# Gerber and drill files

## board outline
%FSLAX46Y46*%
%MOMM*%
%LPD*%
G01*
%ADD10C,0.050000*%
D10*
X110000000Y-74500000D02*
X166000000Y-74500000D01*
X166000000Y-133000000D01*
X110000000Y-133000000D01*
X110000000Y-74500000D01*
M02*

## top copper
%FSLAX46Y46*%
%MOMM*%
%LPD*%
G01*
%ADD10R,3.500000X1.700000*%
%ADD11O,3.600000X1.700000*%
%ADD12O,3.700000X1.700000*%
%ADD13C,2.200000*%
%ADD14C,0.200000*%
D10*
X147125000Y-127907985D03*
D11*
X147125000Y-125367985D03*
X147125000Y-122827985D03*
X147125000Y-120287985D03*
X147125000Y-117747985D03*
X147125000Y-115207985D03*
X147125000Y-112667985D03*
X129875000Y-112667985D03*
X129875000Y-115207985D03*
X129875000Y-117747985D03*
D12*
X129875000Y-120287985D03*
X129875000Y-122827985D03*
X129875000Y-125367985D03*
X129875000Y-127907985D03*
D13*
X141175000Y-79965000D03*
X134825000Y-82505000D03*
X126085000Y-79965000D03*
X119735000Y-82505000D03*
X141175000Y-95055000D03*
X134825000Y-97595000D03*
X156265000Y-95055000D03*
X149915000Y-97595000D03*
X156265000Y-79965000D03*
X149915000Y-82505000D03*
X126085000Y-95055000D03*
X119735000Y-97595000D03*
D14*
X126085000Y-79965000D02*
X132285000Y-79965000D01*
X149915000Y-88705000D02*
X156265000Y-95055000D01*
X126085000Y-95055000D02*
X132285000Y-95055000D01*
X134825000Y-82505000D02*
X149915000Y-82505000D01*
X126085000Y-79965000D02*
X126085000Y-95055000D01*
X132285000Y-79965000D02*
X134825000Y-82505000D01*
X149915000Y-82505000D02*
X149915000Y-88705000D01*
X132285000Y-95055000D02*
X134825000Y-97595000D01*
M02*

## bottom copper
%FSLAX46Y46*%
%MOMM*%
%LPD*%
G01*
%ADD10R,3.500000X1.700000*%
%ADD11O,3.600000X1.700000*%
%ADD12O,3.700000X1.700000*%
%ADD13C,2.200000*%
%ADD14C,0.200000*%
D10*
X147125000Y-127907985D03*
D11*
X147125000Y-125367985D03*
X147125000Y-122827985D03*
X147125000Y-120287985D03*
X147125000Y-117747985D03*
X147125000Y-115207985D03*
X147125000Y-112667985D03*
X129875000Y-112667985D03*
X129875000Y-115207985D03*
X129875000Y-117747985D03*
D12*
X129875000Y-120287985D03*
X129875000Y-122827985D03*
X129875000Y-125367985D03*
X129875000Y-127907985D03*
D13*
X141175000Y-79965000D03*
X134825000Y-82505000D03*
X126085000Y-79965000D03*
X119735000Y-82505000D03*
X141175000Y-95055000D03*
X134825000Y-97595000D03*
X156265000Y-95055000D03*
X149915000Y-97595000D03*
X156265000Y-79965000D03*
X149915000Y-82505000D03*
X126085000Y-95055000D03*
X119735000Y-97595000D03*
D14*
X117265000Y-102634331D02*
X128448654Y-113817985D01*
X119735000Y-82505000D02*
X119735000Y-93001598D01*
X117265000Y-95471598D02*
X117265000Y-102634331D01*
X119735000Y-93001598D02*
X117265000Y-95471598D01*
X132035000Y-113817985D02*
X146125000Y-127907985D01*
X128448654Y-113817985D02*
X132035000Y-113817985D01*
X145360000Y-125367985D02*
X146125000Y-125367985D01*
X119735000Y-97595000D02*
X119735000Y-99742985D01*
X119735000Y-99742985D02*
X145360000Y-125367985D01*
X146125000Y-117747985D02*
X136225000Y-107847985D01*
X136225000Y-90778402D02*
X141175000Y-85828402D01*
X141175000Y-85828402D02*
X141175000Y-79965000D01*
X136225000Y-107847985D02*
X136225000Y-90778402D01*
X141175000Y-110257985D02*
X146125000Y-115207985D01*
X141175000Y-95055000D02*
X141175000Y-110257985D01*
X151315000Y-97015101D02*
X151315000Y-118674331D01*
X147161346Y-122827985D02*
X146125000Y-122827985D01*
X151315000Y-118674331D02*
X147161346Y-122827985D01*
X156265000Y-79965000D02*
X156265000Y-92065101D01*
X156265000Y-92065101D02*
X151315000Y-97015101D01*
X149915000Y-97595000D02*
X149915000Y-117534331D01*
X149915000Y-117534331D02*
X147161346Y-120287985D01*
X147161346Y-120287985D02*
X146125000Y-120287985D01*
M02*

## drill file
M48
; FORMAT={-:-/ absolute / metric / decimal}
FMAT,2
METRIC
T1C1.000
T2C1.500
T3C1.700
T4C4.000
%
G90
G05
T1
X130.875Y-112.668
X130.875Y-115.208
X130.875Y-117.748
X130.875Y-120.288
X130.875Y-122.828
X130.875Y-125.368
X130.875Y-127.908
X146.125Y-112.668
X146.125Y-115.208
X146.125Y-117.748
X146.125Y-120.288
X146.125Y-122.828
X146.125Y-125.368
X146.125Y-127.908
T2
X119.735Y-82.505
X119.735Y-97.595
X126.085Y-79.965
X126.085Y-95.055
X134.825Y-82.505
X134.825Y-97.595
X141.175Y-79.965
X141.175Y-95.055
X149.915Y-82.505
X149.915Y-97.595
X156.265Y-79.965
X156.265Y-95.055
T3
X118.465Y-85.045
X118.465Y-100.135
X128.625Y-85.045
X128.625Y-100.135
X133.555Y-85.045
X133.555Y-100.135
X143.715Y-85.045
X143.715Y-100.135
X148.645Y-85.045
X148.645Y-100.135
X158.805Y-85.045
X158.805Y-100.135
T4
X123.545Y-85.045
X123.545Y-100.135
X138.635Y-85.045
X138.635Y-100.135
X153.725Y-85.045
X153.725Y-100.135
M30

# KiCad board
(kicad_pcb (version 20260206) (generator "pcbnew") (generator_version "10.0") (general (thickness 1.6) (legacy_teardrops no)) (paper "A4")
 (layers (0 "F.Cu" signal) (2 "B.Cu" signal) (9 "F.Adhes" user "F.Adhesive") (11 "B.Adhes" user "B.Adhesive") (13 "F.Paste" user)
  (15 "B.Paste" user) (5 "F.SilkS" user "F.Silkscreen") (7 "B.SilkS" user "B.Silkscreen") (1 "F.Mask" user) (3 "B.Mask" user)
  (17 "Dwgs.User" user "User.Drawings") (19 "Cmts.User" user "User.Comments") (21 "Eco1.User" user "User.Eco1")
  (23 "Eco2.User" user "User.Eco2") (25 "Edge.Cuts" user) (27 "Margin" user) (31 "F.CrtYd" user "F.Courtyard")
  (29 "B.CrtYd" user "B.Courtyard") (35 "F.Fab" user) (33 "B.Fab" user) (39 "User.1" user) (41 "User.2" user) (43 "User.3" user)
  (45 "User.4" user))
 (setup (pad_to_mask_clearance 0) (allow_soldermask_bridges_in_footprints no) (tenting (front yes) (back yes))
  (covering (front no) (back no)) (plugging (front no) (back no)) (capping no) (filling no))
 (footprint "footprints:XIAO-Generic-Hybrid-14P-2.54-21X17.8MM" (layer "F.Cu") (at 138.5 120.287985 180)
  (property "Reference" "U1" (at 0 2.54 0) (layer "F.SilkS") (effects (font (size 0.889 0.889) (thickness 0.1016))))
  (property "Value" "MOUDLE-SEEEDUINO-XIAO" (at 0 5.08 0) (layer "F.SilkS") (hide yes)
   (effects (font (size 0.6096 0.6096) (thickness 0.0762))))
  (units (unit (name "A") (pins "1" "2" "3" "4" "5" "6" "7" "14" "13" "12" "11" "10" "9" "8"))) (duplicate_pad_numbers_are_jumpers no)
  (pad "1" thru_hole rect (at -7.625 -7.62 180) (size 3.5 1.7) (drill 1 (offset -1 0)) (layers "*.Cu" "*.Mask") (remove_unused_layers no)
   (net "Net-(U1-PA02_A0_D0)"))
  (pad "2" thru_hole oval (at -7.625 -5.08 180) (size 3.6 1.7) (drill 1 (offset -1 0)) (layers "*.Cu" "*.Mask") (remove_unused_layers no)
   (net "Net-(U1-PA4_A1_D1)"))
  (pad "3" thru_hole oval (at -7.625 -2.54 180) (size 3.6 1.7) (drill 1 (offset -1 0)) (layers "*.Cu" "*.Mask") (remove_unused_layers no)
   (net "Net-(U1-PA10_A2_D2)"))
  (pad "4" thru_hole oval (at -7.625 0 180) (size 3.6 1.7) (drill 1 (offset -1 0)) (layers "*.Cu" "*.Mask") (remove_unused_layers no)
   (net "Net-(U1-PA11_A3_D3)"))
  (pad "5" thru_hole oval (at -7.625 2.54 180) (size 3.6 1.7) (drill 1 (offset -1 0)) (layers "*.Cu" "*.Mask") (remove_unused_layers no)
   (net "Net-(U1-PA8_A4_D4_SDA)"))
  (pad "6" thru_hole oval (at -7.625 5.08) (size 3.6 1.7) (drill 1 (offset 1 0)) (layers "*.Cu" "*.Mask") (remove_unused_layers no)
   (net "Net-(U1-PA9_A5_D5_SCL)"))
  (pad "7" thru_hole oval (at -7.625 7.62 180) (size 3.6 1.7) (drill 1 (offset -1 0)) (layers "*.Cu" "*.Mask") (remove_unused_layers no)
   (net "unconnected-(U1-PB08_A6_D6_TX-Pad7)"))
  (pad "8" thru_hole oval (at 7.625 7.62 180) (size 3.6 1.7) (drill 1 (offset 1 0)) (layers "*.Cu" "*.Mask") (remove_unused_layers no)
   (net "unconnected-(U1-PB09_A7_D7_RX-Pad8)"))
  (pad "9" thru_hole oval (at 7.625 5.08 180) (size 3.6 1.7) (drill 1 (offset 1 0)) (layers "*.Cu" "*.Mask") (remove_unused_layers no)
   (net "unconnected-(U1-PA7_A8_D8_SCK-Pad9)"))
  (pad "10" thru_hole oval (at 7.625 2.54 180) (size 3.6 1.7) (drill 1 (offset 1 0)) (layers "*.Cu" "*.Mask") (remove_unused_layers no)
   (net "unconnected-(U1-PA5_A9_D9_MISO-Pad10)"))
  (pad "11" thru_hole oval (at 7.625 0 180) (size 3.7 1.7) (drill 1 (offset 1 0)) (layers "*.Cu" "*.Mask") (remove_unused_layers no)
   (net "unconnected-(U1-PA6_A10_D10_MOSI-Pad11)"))
  (pad "12" thru_hole oval (at 7.625 -2.54 180) (size 3.7 1.7) (drill 1 (offset 1 0)) (layers "*.Cu" "*.Mask") (remove_unused_layers no)
   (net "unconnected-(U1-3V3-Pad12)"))
  (pad "13" thru_hole oval (at 7.625 -5.08 180) (size 3.7 1.7) (drill 1 (offset 1 0)) (layers "*.Cu" "*.Mask") (remove_unused_layers no)
   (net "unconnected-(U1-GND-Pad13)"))
  (pad "14" thru_hole oval (at 7.625 -7.62 180) (size 3.7 1.7) (drill 1 (offset 1 0)) (layers "*.Cu" "*.Mask") (remove_unused_layers no)
   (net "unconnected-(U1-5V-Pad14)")))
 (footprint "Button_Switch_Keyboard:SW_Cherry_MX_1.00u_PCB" (layer "F.Cu") (at 141.175 79.965)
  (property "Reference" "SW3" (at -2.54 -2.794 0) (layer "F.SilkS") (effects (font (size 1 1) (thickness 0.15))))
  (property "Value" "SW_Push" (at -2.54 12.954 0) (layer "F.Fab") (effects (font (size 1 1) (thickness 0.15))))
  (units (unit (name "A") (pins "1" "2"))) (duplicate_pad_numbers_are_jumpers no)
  (pad "" np_thru_hole circle (at -7.62 5.08) (size 1.7 1.7) (drill 1.7) (layers "*.Cu" "*.Mask"))
  (pad "" np_thru_hole circle (at -2.54 5.08) (size 4 4) (drill 4) (layers "*.Cu" "*.Mask"))
  (pad "" np_thru_hole circle (at 2.54 5.08) (size 1.7 1.7) (drill 1.7) (layers "*.Cu" "*.Mask"))
  (pad "1" thru_hole circle (at 0 0) (size 2.2 2.2) (drill 1.5) (layers "*.Cu" "*.Mask") (remove_unused_layers no)
   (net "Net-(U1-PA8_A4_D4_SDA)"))
  (pad "2" thru_hole circle (at -6.35 2.54) (size 2.2 2.2) (drill 1.5) (layers "*.Cu" "*.Mask") (remove_unused_layers no) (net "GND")))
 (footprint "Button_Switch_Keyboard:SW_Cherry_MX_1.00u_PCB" (layer "F.Cu") (at 126.085 79.965)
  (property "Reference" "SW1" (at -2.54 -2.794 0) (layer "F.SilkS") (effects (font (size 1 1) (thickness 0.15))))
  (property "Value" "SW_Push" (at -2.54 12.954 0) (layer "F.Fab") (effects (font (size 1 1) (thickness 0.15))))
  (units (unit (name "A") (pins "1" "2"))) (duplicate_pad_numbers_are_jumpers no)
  (pad "" np_thru_hole circle (at -7.62 5.08) (size 1.7 1.7) (drill 1.7) (layers "*.Cu" "*.Mask"))
  (pad "" np_thru_hole circle (at -2.54 5.08) (size 4 4) (drill 4) (layers "*.Cu" "*.Mask"))
  (pad "" np_thru_hole circle (at 2.54 5.08) (size 1.7 1.7) (drill 1.7) (layers "*.Cu" "*.Mask"))
  (pad "1" thru_hole circle (at 0 0) (size 2.2 2.2) (drill 1.5) (layers "*.Cu" "*.Mask") (remove_unused_layers no) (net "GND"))
  (pad "2" thru_hole circle (at -6.35 2.54) (size 2.2 2.2) (drill 1.5) (layers "*.Cu" "*.Mask") (remove_unused_layers no)
   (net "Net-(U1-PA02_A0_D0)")))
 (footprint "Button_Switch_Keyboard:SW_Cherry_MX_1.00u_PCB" (layer "F.Cu") (at 141.175 95.055)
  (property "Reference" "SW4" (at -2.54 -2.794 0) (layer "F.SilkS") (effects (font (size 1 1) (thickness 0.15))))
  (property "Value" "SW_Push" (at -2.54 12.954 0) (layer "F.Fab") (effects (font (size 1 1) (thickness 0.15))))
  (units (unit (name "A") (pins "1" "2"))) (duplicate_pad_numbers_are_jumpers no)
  (pad "" np_thru_hole circle (at -7.62 5.08) (size 1.7 1.7) (drill 1.7) (layers "*.Cu" "*.Mask"))
  (pad "" np_thru_hole circle (at -2.54 5.08) (size 4 4) (drill 4) (layers "*.Cu" "*.Mask"))
  (pad "" np_thru_hole circle (at 2.54 5.08) (size 1.7 1.7) (drill 1.7) (layers "*.Cu" "*.Mask"))
  (pad "1" thru_hole circle (at 0 0) (size 2.2 2.2) (drill 1.5) (layers "*.Cu" "*.Mask") (remove_unused_layers no)
   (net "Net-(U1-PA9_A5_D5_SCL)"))
  (pad "2" thru_hole circle (at -6.35 2.54) (size 2.2 2.2) (drill 1.5) (layers "*.Cu" "*.Mask") (remove_unused_layers no) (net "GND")))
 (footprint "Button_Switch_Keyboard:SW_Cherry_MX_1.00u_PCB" (layer "F.Cu") (at 156.265 95.055)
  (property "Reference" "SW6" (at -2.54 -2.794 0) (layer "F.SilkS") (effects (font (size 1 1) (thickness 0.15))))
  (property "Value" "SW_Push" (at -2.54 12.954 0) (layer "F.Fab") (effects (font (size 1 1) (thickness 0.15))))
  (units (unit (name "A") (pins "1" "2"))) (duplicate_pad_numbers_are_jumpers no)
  (pad "" np_thru_hole circle (at -7.62 5.08) (size 1.7 1.7) (drill 1.7) (layers "*.Cu" "*.Mask"))
  (pad "" np_thru_hole circle (at -2.54 5.08) (size 4 4) (drill 4) (layers "*.Cu" "*.Mask"))
  (pad "" np_thru_hole circle (at 2.54 5.08) (size 1.7 1.7) (drill 1.7) (layers "*.Cu" "*.Mask"))
  (pad "1" thru_hole circle (at 0 0) (size 2.2 2.2) (drill 1.5) (layers "*.Cu" "*.Mask") (remove_unused_layers no) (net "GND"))
  (pad "2" thru_hole circle (at -6.35 2.54) (size 2.2 2.2) (drill 1.5) (layers "*.Cu" "*.Mask") (remove_unused_layers no)
   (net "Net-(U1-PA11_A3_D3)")))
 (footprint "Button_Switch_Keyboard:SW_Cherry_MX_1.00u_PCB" (layer "F.Cu") (at 156.265 79.965)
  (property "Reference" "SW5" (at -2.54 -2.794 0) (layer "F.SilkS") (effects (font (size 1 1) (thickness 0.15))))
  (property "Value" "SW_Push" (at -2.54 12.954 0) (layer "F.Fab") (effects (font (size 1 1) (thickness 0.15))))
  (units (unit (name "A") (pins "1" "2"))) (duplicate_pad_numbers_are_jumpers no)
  (pad "" np_thru_hole circle (at -7.62 5.08) (size 1.7 1.7) (drill 1.7) (layers "*.Cu" "*.Mask"))
  (pad "" np_thru_hole circle (at -2.54 5.08) (size 4 4) (drill 4) (layers "*.Cu" "*.Mask"))
  (pad "" np_thru_hole circle (at 2.54 5.08) (size 1.7 1.7) (drill 1.7) (layers "*.Cu" "*.Mask"))
  (pad "1" thru_hole circle (at 0 0) (size 2.2 2.2) (drill 1.5) (layers "*.Cu" "*.Mask") (remove_unused_layers no)
   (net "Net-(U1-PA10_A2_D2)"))
  (pad "2" thru_hole circle (at -6.35 2.54) (size 2.2 2.2) (drill 1.5) (layers "*.Cu" "*.Mask") (remove_unused_layers no) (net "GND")))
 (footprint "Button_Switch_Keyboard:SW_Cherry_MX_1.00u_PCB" (layer "F.Cu") (at 126.085 95.055)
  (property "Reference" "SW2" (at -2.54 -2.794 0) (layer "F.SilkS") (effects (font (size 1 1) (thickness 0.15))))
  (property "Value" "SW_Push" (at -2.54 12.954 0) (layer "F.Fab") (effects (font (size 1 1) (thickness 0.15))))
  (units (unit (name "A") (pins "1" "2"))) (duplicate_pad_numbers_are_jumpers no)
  (pad "" np_thru_hole circle (at -7.62 5.08) (size 1.7 1.7) (drill 1.7) (layers "*.Cu" "*.Mask"))
  (pad "" np_thru_hole circle (at -2.54 5.08) (size 4 4) (drill 4) (layers "*.Cu" "*.Mask"))
  (pad "" np_thru_hole circle (at 2.54 5.08) (size 1.7 1.7) (drill 1.7) (layers "*.Cu" "*.Mask"))
  (pad "1" thru_hole circle (at 0 0) (size 2.2 2.2) (drill 1.5) (layers "*.Cu" "*.Mask") (remove_unused_layers no) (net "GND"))
  (pad "2" thru_hole circle (at -6.35 2.54) (size 2.2 2.2) (drill 1.5) (layers "*.Cu" "*.Mask") (remove_unused_layers no)
   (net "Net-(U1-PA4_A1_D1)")))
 (gr_rect (start 110 74.5) (end 166 133) (stroke (width 0.05) (type default)) (fill no) (layer "Edge.Cuts"))
 (segment (start 117.265 102.634331) (end 128.448654 113.817985) (width 0.2) (layer "B.Cu") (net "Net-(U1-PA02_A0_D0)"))
 (segment (start 119.735 82.505) (end 119.735 93.001598) (width 0.2) (layer "B.Cu") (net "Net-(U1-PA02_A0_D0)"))
 (segment (start 117.265 95.471598) (end 117.265 102.634331) (width 0.2) (layer "B.Cu") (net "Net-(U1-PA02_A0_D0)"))
 (segment (start 119.735 93.001598) (end 117.265 95.471598) (width 0.2) (layer "B.Cu") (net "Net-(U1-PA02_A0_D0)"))
 (segment (start 132.035 113.817985) (end 146.125 127.907985) (width 0.2) (layer "B.Cu") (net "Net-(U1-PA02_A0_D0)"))
 (segment (start 128.448654 113.817985) (end 132.035 113.817985) (width 0.2) (layer "B.Cu") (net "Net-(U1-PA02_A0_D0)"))
 (segment (start 126.085 79.965) (end 132.285 79.965) (width 0.2) (layer "F.Cu") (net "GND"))
 (segment (start 149.915 88.705) (end 156.265 95.055) (width 0.2) (layer "F.Cu") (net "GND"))
 (segment (start 126.085 95.055) (end 132.285 95.055) (width 0.2) (layer "F.Cu") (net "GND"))
 (segment (start 134.825 82.505) (end 149.915 82.505) (width 0.2) (layer "F.Cu") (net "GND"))
 (segment (start 126.085 79.965) (end 126.085 95.055) (width 0.2) (layer "F.Cu") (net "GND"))
 (segment (start 132.285 79.965) (end 134.825 82.505) (width 0.2) (layer "F.Cu") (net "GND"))
 (segment (start 149.915 82.505) (end 149.915 88.705) (width 0.2) (layer "F.Cu") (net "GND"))
 (segment (start 132.285 95.055) (end 134.825 97.595) (width 0.2) (layer "F.Cu") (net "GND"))
 (segment (start 145.36 125.367985) (end 146.125 125.367985) (width 0.2) (layer "B.Cu") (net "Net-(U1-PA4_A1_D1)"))
 (segment (start 119.735 97.595) (end 119.735 99.742985) (width 0.2) (layer "B.Cu") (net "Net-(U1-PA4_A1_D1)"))
 (segment (start 119.735 99.742985) (end 145.36 125.367985) (width 0.2) (layer "B.Cu") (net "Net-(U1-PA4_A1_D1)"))
 (segment (start 146.125 117.747985) (end 136.225 107.847985) (width 0.2) (layer "B.Cu") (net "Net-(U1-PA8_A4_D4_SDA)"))
 (segment (start 136.225 90.778402) (end 141.175 85.828402) (width 0.2) (layer "B.Cu") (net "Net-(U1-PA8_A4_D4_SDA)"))
 (segment (start 141.175 85.828402) (end 141.175 79.965) (width 0.2) (layer "B.Cu") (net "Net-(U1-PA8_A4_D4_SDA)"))
 (segment (start 136.225 107.847985) (end 136.225 90.778402) (width 0.2) (layer "B.Cu") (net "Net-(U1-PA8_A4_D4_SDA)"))
 (segment (start 141.175 110.257985) (end 146.125 115.207985) (width 0.2) (layer "B.Cu") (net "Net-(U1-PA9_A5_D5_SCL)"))
 (segment (start 141.175 95.055) (end 141.175 110.257985) (width 0.2) (layer "B.Cu") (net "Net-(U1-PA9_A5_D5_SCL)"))
 (segment (start 151.315 97.015101) (end 151.315 118.674331) (width 0.2) (layer "B.Cu") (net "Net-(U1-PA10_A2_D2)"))
 (segment (start 147.161346 122.827985) (end 146.125 122.827985) (width 0.2) (layer "B.Cu") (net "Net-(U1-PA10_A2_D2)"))
 (segment (start 151.315 118.674331) (end 147.161346 122.827985) (width 0.2) (layer "B.Cu") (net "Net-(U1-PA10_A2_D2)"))
 (segment (start 156.265 79.965) (end 156.265 92.065101) (width 0.2) (layer "B.Cu") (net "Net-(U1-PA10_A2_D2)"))
 (segment (start 156.265 92.065101) (end 151.315 97.015101) (width 0.2) (layer "B.Cu") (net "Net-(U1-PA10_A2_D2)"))
 (segment (start 149.915 97.595) (end 149.915 117.534331) (width 0.2) (layer "B.Cu") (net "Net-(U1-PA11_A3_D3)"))
 (segment (start 149.915 117.534331) (end 147.161346 120.287985) (width 0.2) (layer "B.Cu") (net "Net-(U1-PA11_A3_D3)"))
 (segment (start 147.161346 120.287985) (end 146.125 120.287985) (width 0.2) (layer "B.Cu") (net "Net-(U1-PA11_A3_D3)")))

